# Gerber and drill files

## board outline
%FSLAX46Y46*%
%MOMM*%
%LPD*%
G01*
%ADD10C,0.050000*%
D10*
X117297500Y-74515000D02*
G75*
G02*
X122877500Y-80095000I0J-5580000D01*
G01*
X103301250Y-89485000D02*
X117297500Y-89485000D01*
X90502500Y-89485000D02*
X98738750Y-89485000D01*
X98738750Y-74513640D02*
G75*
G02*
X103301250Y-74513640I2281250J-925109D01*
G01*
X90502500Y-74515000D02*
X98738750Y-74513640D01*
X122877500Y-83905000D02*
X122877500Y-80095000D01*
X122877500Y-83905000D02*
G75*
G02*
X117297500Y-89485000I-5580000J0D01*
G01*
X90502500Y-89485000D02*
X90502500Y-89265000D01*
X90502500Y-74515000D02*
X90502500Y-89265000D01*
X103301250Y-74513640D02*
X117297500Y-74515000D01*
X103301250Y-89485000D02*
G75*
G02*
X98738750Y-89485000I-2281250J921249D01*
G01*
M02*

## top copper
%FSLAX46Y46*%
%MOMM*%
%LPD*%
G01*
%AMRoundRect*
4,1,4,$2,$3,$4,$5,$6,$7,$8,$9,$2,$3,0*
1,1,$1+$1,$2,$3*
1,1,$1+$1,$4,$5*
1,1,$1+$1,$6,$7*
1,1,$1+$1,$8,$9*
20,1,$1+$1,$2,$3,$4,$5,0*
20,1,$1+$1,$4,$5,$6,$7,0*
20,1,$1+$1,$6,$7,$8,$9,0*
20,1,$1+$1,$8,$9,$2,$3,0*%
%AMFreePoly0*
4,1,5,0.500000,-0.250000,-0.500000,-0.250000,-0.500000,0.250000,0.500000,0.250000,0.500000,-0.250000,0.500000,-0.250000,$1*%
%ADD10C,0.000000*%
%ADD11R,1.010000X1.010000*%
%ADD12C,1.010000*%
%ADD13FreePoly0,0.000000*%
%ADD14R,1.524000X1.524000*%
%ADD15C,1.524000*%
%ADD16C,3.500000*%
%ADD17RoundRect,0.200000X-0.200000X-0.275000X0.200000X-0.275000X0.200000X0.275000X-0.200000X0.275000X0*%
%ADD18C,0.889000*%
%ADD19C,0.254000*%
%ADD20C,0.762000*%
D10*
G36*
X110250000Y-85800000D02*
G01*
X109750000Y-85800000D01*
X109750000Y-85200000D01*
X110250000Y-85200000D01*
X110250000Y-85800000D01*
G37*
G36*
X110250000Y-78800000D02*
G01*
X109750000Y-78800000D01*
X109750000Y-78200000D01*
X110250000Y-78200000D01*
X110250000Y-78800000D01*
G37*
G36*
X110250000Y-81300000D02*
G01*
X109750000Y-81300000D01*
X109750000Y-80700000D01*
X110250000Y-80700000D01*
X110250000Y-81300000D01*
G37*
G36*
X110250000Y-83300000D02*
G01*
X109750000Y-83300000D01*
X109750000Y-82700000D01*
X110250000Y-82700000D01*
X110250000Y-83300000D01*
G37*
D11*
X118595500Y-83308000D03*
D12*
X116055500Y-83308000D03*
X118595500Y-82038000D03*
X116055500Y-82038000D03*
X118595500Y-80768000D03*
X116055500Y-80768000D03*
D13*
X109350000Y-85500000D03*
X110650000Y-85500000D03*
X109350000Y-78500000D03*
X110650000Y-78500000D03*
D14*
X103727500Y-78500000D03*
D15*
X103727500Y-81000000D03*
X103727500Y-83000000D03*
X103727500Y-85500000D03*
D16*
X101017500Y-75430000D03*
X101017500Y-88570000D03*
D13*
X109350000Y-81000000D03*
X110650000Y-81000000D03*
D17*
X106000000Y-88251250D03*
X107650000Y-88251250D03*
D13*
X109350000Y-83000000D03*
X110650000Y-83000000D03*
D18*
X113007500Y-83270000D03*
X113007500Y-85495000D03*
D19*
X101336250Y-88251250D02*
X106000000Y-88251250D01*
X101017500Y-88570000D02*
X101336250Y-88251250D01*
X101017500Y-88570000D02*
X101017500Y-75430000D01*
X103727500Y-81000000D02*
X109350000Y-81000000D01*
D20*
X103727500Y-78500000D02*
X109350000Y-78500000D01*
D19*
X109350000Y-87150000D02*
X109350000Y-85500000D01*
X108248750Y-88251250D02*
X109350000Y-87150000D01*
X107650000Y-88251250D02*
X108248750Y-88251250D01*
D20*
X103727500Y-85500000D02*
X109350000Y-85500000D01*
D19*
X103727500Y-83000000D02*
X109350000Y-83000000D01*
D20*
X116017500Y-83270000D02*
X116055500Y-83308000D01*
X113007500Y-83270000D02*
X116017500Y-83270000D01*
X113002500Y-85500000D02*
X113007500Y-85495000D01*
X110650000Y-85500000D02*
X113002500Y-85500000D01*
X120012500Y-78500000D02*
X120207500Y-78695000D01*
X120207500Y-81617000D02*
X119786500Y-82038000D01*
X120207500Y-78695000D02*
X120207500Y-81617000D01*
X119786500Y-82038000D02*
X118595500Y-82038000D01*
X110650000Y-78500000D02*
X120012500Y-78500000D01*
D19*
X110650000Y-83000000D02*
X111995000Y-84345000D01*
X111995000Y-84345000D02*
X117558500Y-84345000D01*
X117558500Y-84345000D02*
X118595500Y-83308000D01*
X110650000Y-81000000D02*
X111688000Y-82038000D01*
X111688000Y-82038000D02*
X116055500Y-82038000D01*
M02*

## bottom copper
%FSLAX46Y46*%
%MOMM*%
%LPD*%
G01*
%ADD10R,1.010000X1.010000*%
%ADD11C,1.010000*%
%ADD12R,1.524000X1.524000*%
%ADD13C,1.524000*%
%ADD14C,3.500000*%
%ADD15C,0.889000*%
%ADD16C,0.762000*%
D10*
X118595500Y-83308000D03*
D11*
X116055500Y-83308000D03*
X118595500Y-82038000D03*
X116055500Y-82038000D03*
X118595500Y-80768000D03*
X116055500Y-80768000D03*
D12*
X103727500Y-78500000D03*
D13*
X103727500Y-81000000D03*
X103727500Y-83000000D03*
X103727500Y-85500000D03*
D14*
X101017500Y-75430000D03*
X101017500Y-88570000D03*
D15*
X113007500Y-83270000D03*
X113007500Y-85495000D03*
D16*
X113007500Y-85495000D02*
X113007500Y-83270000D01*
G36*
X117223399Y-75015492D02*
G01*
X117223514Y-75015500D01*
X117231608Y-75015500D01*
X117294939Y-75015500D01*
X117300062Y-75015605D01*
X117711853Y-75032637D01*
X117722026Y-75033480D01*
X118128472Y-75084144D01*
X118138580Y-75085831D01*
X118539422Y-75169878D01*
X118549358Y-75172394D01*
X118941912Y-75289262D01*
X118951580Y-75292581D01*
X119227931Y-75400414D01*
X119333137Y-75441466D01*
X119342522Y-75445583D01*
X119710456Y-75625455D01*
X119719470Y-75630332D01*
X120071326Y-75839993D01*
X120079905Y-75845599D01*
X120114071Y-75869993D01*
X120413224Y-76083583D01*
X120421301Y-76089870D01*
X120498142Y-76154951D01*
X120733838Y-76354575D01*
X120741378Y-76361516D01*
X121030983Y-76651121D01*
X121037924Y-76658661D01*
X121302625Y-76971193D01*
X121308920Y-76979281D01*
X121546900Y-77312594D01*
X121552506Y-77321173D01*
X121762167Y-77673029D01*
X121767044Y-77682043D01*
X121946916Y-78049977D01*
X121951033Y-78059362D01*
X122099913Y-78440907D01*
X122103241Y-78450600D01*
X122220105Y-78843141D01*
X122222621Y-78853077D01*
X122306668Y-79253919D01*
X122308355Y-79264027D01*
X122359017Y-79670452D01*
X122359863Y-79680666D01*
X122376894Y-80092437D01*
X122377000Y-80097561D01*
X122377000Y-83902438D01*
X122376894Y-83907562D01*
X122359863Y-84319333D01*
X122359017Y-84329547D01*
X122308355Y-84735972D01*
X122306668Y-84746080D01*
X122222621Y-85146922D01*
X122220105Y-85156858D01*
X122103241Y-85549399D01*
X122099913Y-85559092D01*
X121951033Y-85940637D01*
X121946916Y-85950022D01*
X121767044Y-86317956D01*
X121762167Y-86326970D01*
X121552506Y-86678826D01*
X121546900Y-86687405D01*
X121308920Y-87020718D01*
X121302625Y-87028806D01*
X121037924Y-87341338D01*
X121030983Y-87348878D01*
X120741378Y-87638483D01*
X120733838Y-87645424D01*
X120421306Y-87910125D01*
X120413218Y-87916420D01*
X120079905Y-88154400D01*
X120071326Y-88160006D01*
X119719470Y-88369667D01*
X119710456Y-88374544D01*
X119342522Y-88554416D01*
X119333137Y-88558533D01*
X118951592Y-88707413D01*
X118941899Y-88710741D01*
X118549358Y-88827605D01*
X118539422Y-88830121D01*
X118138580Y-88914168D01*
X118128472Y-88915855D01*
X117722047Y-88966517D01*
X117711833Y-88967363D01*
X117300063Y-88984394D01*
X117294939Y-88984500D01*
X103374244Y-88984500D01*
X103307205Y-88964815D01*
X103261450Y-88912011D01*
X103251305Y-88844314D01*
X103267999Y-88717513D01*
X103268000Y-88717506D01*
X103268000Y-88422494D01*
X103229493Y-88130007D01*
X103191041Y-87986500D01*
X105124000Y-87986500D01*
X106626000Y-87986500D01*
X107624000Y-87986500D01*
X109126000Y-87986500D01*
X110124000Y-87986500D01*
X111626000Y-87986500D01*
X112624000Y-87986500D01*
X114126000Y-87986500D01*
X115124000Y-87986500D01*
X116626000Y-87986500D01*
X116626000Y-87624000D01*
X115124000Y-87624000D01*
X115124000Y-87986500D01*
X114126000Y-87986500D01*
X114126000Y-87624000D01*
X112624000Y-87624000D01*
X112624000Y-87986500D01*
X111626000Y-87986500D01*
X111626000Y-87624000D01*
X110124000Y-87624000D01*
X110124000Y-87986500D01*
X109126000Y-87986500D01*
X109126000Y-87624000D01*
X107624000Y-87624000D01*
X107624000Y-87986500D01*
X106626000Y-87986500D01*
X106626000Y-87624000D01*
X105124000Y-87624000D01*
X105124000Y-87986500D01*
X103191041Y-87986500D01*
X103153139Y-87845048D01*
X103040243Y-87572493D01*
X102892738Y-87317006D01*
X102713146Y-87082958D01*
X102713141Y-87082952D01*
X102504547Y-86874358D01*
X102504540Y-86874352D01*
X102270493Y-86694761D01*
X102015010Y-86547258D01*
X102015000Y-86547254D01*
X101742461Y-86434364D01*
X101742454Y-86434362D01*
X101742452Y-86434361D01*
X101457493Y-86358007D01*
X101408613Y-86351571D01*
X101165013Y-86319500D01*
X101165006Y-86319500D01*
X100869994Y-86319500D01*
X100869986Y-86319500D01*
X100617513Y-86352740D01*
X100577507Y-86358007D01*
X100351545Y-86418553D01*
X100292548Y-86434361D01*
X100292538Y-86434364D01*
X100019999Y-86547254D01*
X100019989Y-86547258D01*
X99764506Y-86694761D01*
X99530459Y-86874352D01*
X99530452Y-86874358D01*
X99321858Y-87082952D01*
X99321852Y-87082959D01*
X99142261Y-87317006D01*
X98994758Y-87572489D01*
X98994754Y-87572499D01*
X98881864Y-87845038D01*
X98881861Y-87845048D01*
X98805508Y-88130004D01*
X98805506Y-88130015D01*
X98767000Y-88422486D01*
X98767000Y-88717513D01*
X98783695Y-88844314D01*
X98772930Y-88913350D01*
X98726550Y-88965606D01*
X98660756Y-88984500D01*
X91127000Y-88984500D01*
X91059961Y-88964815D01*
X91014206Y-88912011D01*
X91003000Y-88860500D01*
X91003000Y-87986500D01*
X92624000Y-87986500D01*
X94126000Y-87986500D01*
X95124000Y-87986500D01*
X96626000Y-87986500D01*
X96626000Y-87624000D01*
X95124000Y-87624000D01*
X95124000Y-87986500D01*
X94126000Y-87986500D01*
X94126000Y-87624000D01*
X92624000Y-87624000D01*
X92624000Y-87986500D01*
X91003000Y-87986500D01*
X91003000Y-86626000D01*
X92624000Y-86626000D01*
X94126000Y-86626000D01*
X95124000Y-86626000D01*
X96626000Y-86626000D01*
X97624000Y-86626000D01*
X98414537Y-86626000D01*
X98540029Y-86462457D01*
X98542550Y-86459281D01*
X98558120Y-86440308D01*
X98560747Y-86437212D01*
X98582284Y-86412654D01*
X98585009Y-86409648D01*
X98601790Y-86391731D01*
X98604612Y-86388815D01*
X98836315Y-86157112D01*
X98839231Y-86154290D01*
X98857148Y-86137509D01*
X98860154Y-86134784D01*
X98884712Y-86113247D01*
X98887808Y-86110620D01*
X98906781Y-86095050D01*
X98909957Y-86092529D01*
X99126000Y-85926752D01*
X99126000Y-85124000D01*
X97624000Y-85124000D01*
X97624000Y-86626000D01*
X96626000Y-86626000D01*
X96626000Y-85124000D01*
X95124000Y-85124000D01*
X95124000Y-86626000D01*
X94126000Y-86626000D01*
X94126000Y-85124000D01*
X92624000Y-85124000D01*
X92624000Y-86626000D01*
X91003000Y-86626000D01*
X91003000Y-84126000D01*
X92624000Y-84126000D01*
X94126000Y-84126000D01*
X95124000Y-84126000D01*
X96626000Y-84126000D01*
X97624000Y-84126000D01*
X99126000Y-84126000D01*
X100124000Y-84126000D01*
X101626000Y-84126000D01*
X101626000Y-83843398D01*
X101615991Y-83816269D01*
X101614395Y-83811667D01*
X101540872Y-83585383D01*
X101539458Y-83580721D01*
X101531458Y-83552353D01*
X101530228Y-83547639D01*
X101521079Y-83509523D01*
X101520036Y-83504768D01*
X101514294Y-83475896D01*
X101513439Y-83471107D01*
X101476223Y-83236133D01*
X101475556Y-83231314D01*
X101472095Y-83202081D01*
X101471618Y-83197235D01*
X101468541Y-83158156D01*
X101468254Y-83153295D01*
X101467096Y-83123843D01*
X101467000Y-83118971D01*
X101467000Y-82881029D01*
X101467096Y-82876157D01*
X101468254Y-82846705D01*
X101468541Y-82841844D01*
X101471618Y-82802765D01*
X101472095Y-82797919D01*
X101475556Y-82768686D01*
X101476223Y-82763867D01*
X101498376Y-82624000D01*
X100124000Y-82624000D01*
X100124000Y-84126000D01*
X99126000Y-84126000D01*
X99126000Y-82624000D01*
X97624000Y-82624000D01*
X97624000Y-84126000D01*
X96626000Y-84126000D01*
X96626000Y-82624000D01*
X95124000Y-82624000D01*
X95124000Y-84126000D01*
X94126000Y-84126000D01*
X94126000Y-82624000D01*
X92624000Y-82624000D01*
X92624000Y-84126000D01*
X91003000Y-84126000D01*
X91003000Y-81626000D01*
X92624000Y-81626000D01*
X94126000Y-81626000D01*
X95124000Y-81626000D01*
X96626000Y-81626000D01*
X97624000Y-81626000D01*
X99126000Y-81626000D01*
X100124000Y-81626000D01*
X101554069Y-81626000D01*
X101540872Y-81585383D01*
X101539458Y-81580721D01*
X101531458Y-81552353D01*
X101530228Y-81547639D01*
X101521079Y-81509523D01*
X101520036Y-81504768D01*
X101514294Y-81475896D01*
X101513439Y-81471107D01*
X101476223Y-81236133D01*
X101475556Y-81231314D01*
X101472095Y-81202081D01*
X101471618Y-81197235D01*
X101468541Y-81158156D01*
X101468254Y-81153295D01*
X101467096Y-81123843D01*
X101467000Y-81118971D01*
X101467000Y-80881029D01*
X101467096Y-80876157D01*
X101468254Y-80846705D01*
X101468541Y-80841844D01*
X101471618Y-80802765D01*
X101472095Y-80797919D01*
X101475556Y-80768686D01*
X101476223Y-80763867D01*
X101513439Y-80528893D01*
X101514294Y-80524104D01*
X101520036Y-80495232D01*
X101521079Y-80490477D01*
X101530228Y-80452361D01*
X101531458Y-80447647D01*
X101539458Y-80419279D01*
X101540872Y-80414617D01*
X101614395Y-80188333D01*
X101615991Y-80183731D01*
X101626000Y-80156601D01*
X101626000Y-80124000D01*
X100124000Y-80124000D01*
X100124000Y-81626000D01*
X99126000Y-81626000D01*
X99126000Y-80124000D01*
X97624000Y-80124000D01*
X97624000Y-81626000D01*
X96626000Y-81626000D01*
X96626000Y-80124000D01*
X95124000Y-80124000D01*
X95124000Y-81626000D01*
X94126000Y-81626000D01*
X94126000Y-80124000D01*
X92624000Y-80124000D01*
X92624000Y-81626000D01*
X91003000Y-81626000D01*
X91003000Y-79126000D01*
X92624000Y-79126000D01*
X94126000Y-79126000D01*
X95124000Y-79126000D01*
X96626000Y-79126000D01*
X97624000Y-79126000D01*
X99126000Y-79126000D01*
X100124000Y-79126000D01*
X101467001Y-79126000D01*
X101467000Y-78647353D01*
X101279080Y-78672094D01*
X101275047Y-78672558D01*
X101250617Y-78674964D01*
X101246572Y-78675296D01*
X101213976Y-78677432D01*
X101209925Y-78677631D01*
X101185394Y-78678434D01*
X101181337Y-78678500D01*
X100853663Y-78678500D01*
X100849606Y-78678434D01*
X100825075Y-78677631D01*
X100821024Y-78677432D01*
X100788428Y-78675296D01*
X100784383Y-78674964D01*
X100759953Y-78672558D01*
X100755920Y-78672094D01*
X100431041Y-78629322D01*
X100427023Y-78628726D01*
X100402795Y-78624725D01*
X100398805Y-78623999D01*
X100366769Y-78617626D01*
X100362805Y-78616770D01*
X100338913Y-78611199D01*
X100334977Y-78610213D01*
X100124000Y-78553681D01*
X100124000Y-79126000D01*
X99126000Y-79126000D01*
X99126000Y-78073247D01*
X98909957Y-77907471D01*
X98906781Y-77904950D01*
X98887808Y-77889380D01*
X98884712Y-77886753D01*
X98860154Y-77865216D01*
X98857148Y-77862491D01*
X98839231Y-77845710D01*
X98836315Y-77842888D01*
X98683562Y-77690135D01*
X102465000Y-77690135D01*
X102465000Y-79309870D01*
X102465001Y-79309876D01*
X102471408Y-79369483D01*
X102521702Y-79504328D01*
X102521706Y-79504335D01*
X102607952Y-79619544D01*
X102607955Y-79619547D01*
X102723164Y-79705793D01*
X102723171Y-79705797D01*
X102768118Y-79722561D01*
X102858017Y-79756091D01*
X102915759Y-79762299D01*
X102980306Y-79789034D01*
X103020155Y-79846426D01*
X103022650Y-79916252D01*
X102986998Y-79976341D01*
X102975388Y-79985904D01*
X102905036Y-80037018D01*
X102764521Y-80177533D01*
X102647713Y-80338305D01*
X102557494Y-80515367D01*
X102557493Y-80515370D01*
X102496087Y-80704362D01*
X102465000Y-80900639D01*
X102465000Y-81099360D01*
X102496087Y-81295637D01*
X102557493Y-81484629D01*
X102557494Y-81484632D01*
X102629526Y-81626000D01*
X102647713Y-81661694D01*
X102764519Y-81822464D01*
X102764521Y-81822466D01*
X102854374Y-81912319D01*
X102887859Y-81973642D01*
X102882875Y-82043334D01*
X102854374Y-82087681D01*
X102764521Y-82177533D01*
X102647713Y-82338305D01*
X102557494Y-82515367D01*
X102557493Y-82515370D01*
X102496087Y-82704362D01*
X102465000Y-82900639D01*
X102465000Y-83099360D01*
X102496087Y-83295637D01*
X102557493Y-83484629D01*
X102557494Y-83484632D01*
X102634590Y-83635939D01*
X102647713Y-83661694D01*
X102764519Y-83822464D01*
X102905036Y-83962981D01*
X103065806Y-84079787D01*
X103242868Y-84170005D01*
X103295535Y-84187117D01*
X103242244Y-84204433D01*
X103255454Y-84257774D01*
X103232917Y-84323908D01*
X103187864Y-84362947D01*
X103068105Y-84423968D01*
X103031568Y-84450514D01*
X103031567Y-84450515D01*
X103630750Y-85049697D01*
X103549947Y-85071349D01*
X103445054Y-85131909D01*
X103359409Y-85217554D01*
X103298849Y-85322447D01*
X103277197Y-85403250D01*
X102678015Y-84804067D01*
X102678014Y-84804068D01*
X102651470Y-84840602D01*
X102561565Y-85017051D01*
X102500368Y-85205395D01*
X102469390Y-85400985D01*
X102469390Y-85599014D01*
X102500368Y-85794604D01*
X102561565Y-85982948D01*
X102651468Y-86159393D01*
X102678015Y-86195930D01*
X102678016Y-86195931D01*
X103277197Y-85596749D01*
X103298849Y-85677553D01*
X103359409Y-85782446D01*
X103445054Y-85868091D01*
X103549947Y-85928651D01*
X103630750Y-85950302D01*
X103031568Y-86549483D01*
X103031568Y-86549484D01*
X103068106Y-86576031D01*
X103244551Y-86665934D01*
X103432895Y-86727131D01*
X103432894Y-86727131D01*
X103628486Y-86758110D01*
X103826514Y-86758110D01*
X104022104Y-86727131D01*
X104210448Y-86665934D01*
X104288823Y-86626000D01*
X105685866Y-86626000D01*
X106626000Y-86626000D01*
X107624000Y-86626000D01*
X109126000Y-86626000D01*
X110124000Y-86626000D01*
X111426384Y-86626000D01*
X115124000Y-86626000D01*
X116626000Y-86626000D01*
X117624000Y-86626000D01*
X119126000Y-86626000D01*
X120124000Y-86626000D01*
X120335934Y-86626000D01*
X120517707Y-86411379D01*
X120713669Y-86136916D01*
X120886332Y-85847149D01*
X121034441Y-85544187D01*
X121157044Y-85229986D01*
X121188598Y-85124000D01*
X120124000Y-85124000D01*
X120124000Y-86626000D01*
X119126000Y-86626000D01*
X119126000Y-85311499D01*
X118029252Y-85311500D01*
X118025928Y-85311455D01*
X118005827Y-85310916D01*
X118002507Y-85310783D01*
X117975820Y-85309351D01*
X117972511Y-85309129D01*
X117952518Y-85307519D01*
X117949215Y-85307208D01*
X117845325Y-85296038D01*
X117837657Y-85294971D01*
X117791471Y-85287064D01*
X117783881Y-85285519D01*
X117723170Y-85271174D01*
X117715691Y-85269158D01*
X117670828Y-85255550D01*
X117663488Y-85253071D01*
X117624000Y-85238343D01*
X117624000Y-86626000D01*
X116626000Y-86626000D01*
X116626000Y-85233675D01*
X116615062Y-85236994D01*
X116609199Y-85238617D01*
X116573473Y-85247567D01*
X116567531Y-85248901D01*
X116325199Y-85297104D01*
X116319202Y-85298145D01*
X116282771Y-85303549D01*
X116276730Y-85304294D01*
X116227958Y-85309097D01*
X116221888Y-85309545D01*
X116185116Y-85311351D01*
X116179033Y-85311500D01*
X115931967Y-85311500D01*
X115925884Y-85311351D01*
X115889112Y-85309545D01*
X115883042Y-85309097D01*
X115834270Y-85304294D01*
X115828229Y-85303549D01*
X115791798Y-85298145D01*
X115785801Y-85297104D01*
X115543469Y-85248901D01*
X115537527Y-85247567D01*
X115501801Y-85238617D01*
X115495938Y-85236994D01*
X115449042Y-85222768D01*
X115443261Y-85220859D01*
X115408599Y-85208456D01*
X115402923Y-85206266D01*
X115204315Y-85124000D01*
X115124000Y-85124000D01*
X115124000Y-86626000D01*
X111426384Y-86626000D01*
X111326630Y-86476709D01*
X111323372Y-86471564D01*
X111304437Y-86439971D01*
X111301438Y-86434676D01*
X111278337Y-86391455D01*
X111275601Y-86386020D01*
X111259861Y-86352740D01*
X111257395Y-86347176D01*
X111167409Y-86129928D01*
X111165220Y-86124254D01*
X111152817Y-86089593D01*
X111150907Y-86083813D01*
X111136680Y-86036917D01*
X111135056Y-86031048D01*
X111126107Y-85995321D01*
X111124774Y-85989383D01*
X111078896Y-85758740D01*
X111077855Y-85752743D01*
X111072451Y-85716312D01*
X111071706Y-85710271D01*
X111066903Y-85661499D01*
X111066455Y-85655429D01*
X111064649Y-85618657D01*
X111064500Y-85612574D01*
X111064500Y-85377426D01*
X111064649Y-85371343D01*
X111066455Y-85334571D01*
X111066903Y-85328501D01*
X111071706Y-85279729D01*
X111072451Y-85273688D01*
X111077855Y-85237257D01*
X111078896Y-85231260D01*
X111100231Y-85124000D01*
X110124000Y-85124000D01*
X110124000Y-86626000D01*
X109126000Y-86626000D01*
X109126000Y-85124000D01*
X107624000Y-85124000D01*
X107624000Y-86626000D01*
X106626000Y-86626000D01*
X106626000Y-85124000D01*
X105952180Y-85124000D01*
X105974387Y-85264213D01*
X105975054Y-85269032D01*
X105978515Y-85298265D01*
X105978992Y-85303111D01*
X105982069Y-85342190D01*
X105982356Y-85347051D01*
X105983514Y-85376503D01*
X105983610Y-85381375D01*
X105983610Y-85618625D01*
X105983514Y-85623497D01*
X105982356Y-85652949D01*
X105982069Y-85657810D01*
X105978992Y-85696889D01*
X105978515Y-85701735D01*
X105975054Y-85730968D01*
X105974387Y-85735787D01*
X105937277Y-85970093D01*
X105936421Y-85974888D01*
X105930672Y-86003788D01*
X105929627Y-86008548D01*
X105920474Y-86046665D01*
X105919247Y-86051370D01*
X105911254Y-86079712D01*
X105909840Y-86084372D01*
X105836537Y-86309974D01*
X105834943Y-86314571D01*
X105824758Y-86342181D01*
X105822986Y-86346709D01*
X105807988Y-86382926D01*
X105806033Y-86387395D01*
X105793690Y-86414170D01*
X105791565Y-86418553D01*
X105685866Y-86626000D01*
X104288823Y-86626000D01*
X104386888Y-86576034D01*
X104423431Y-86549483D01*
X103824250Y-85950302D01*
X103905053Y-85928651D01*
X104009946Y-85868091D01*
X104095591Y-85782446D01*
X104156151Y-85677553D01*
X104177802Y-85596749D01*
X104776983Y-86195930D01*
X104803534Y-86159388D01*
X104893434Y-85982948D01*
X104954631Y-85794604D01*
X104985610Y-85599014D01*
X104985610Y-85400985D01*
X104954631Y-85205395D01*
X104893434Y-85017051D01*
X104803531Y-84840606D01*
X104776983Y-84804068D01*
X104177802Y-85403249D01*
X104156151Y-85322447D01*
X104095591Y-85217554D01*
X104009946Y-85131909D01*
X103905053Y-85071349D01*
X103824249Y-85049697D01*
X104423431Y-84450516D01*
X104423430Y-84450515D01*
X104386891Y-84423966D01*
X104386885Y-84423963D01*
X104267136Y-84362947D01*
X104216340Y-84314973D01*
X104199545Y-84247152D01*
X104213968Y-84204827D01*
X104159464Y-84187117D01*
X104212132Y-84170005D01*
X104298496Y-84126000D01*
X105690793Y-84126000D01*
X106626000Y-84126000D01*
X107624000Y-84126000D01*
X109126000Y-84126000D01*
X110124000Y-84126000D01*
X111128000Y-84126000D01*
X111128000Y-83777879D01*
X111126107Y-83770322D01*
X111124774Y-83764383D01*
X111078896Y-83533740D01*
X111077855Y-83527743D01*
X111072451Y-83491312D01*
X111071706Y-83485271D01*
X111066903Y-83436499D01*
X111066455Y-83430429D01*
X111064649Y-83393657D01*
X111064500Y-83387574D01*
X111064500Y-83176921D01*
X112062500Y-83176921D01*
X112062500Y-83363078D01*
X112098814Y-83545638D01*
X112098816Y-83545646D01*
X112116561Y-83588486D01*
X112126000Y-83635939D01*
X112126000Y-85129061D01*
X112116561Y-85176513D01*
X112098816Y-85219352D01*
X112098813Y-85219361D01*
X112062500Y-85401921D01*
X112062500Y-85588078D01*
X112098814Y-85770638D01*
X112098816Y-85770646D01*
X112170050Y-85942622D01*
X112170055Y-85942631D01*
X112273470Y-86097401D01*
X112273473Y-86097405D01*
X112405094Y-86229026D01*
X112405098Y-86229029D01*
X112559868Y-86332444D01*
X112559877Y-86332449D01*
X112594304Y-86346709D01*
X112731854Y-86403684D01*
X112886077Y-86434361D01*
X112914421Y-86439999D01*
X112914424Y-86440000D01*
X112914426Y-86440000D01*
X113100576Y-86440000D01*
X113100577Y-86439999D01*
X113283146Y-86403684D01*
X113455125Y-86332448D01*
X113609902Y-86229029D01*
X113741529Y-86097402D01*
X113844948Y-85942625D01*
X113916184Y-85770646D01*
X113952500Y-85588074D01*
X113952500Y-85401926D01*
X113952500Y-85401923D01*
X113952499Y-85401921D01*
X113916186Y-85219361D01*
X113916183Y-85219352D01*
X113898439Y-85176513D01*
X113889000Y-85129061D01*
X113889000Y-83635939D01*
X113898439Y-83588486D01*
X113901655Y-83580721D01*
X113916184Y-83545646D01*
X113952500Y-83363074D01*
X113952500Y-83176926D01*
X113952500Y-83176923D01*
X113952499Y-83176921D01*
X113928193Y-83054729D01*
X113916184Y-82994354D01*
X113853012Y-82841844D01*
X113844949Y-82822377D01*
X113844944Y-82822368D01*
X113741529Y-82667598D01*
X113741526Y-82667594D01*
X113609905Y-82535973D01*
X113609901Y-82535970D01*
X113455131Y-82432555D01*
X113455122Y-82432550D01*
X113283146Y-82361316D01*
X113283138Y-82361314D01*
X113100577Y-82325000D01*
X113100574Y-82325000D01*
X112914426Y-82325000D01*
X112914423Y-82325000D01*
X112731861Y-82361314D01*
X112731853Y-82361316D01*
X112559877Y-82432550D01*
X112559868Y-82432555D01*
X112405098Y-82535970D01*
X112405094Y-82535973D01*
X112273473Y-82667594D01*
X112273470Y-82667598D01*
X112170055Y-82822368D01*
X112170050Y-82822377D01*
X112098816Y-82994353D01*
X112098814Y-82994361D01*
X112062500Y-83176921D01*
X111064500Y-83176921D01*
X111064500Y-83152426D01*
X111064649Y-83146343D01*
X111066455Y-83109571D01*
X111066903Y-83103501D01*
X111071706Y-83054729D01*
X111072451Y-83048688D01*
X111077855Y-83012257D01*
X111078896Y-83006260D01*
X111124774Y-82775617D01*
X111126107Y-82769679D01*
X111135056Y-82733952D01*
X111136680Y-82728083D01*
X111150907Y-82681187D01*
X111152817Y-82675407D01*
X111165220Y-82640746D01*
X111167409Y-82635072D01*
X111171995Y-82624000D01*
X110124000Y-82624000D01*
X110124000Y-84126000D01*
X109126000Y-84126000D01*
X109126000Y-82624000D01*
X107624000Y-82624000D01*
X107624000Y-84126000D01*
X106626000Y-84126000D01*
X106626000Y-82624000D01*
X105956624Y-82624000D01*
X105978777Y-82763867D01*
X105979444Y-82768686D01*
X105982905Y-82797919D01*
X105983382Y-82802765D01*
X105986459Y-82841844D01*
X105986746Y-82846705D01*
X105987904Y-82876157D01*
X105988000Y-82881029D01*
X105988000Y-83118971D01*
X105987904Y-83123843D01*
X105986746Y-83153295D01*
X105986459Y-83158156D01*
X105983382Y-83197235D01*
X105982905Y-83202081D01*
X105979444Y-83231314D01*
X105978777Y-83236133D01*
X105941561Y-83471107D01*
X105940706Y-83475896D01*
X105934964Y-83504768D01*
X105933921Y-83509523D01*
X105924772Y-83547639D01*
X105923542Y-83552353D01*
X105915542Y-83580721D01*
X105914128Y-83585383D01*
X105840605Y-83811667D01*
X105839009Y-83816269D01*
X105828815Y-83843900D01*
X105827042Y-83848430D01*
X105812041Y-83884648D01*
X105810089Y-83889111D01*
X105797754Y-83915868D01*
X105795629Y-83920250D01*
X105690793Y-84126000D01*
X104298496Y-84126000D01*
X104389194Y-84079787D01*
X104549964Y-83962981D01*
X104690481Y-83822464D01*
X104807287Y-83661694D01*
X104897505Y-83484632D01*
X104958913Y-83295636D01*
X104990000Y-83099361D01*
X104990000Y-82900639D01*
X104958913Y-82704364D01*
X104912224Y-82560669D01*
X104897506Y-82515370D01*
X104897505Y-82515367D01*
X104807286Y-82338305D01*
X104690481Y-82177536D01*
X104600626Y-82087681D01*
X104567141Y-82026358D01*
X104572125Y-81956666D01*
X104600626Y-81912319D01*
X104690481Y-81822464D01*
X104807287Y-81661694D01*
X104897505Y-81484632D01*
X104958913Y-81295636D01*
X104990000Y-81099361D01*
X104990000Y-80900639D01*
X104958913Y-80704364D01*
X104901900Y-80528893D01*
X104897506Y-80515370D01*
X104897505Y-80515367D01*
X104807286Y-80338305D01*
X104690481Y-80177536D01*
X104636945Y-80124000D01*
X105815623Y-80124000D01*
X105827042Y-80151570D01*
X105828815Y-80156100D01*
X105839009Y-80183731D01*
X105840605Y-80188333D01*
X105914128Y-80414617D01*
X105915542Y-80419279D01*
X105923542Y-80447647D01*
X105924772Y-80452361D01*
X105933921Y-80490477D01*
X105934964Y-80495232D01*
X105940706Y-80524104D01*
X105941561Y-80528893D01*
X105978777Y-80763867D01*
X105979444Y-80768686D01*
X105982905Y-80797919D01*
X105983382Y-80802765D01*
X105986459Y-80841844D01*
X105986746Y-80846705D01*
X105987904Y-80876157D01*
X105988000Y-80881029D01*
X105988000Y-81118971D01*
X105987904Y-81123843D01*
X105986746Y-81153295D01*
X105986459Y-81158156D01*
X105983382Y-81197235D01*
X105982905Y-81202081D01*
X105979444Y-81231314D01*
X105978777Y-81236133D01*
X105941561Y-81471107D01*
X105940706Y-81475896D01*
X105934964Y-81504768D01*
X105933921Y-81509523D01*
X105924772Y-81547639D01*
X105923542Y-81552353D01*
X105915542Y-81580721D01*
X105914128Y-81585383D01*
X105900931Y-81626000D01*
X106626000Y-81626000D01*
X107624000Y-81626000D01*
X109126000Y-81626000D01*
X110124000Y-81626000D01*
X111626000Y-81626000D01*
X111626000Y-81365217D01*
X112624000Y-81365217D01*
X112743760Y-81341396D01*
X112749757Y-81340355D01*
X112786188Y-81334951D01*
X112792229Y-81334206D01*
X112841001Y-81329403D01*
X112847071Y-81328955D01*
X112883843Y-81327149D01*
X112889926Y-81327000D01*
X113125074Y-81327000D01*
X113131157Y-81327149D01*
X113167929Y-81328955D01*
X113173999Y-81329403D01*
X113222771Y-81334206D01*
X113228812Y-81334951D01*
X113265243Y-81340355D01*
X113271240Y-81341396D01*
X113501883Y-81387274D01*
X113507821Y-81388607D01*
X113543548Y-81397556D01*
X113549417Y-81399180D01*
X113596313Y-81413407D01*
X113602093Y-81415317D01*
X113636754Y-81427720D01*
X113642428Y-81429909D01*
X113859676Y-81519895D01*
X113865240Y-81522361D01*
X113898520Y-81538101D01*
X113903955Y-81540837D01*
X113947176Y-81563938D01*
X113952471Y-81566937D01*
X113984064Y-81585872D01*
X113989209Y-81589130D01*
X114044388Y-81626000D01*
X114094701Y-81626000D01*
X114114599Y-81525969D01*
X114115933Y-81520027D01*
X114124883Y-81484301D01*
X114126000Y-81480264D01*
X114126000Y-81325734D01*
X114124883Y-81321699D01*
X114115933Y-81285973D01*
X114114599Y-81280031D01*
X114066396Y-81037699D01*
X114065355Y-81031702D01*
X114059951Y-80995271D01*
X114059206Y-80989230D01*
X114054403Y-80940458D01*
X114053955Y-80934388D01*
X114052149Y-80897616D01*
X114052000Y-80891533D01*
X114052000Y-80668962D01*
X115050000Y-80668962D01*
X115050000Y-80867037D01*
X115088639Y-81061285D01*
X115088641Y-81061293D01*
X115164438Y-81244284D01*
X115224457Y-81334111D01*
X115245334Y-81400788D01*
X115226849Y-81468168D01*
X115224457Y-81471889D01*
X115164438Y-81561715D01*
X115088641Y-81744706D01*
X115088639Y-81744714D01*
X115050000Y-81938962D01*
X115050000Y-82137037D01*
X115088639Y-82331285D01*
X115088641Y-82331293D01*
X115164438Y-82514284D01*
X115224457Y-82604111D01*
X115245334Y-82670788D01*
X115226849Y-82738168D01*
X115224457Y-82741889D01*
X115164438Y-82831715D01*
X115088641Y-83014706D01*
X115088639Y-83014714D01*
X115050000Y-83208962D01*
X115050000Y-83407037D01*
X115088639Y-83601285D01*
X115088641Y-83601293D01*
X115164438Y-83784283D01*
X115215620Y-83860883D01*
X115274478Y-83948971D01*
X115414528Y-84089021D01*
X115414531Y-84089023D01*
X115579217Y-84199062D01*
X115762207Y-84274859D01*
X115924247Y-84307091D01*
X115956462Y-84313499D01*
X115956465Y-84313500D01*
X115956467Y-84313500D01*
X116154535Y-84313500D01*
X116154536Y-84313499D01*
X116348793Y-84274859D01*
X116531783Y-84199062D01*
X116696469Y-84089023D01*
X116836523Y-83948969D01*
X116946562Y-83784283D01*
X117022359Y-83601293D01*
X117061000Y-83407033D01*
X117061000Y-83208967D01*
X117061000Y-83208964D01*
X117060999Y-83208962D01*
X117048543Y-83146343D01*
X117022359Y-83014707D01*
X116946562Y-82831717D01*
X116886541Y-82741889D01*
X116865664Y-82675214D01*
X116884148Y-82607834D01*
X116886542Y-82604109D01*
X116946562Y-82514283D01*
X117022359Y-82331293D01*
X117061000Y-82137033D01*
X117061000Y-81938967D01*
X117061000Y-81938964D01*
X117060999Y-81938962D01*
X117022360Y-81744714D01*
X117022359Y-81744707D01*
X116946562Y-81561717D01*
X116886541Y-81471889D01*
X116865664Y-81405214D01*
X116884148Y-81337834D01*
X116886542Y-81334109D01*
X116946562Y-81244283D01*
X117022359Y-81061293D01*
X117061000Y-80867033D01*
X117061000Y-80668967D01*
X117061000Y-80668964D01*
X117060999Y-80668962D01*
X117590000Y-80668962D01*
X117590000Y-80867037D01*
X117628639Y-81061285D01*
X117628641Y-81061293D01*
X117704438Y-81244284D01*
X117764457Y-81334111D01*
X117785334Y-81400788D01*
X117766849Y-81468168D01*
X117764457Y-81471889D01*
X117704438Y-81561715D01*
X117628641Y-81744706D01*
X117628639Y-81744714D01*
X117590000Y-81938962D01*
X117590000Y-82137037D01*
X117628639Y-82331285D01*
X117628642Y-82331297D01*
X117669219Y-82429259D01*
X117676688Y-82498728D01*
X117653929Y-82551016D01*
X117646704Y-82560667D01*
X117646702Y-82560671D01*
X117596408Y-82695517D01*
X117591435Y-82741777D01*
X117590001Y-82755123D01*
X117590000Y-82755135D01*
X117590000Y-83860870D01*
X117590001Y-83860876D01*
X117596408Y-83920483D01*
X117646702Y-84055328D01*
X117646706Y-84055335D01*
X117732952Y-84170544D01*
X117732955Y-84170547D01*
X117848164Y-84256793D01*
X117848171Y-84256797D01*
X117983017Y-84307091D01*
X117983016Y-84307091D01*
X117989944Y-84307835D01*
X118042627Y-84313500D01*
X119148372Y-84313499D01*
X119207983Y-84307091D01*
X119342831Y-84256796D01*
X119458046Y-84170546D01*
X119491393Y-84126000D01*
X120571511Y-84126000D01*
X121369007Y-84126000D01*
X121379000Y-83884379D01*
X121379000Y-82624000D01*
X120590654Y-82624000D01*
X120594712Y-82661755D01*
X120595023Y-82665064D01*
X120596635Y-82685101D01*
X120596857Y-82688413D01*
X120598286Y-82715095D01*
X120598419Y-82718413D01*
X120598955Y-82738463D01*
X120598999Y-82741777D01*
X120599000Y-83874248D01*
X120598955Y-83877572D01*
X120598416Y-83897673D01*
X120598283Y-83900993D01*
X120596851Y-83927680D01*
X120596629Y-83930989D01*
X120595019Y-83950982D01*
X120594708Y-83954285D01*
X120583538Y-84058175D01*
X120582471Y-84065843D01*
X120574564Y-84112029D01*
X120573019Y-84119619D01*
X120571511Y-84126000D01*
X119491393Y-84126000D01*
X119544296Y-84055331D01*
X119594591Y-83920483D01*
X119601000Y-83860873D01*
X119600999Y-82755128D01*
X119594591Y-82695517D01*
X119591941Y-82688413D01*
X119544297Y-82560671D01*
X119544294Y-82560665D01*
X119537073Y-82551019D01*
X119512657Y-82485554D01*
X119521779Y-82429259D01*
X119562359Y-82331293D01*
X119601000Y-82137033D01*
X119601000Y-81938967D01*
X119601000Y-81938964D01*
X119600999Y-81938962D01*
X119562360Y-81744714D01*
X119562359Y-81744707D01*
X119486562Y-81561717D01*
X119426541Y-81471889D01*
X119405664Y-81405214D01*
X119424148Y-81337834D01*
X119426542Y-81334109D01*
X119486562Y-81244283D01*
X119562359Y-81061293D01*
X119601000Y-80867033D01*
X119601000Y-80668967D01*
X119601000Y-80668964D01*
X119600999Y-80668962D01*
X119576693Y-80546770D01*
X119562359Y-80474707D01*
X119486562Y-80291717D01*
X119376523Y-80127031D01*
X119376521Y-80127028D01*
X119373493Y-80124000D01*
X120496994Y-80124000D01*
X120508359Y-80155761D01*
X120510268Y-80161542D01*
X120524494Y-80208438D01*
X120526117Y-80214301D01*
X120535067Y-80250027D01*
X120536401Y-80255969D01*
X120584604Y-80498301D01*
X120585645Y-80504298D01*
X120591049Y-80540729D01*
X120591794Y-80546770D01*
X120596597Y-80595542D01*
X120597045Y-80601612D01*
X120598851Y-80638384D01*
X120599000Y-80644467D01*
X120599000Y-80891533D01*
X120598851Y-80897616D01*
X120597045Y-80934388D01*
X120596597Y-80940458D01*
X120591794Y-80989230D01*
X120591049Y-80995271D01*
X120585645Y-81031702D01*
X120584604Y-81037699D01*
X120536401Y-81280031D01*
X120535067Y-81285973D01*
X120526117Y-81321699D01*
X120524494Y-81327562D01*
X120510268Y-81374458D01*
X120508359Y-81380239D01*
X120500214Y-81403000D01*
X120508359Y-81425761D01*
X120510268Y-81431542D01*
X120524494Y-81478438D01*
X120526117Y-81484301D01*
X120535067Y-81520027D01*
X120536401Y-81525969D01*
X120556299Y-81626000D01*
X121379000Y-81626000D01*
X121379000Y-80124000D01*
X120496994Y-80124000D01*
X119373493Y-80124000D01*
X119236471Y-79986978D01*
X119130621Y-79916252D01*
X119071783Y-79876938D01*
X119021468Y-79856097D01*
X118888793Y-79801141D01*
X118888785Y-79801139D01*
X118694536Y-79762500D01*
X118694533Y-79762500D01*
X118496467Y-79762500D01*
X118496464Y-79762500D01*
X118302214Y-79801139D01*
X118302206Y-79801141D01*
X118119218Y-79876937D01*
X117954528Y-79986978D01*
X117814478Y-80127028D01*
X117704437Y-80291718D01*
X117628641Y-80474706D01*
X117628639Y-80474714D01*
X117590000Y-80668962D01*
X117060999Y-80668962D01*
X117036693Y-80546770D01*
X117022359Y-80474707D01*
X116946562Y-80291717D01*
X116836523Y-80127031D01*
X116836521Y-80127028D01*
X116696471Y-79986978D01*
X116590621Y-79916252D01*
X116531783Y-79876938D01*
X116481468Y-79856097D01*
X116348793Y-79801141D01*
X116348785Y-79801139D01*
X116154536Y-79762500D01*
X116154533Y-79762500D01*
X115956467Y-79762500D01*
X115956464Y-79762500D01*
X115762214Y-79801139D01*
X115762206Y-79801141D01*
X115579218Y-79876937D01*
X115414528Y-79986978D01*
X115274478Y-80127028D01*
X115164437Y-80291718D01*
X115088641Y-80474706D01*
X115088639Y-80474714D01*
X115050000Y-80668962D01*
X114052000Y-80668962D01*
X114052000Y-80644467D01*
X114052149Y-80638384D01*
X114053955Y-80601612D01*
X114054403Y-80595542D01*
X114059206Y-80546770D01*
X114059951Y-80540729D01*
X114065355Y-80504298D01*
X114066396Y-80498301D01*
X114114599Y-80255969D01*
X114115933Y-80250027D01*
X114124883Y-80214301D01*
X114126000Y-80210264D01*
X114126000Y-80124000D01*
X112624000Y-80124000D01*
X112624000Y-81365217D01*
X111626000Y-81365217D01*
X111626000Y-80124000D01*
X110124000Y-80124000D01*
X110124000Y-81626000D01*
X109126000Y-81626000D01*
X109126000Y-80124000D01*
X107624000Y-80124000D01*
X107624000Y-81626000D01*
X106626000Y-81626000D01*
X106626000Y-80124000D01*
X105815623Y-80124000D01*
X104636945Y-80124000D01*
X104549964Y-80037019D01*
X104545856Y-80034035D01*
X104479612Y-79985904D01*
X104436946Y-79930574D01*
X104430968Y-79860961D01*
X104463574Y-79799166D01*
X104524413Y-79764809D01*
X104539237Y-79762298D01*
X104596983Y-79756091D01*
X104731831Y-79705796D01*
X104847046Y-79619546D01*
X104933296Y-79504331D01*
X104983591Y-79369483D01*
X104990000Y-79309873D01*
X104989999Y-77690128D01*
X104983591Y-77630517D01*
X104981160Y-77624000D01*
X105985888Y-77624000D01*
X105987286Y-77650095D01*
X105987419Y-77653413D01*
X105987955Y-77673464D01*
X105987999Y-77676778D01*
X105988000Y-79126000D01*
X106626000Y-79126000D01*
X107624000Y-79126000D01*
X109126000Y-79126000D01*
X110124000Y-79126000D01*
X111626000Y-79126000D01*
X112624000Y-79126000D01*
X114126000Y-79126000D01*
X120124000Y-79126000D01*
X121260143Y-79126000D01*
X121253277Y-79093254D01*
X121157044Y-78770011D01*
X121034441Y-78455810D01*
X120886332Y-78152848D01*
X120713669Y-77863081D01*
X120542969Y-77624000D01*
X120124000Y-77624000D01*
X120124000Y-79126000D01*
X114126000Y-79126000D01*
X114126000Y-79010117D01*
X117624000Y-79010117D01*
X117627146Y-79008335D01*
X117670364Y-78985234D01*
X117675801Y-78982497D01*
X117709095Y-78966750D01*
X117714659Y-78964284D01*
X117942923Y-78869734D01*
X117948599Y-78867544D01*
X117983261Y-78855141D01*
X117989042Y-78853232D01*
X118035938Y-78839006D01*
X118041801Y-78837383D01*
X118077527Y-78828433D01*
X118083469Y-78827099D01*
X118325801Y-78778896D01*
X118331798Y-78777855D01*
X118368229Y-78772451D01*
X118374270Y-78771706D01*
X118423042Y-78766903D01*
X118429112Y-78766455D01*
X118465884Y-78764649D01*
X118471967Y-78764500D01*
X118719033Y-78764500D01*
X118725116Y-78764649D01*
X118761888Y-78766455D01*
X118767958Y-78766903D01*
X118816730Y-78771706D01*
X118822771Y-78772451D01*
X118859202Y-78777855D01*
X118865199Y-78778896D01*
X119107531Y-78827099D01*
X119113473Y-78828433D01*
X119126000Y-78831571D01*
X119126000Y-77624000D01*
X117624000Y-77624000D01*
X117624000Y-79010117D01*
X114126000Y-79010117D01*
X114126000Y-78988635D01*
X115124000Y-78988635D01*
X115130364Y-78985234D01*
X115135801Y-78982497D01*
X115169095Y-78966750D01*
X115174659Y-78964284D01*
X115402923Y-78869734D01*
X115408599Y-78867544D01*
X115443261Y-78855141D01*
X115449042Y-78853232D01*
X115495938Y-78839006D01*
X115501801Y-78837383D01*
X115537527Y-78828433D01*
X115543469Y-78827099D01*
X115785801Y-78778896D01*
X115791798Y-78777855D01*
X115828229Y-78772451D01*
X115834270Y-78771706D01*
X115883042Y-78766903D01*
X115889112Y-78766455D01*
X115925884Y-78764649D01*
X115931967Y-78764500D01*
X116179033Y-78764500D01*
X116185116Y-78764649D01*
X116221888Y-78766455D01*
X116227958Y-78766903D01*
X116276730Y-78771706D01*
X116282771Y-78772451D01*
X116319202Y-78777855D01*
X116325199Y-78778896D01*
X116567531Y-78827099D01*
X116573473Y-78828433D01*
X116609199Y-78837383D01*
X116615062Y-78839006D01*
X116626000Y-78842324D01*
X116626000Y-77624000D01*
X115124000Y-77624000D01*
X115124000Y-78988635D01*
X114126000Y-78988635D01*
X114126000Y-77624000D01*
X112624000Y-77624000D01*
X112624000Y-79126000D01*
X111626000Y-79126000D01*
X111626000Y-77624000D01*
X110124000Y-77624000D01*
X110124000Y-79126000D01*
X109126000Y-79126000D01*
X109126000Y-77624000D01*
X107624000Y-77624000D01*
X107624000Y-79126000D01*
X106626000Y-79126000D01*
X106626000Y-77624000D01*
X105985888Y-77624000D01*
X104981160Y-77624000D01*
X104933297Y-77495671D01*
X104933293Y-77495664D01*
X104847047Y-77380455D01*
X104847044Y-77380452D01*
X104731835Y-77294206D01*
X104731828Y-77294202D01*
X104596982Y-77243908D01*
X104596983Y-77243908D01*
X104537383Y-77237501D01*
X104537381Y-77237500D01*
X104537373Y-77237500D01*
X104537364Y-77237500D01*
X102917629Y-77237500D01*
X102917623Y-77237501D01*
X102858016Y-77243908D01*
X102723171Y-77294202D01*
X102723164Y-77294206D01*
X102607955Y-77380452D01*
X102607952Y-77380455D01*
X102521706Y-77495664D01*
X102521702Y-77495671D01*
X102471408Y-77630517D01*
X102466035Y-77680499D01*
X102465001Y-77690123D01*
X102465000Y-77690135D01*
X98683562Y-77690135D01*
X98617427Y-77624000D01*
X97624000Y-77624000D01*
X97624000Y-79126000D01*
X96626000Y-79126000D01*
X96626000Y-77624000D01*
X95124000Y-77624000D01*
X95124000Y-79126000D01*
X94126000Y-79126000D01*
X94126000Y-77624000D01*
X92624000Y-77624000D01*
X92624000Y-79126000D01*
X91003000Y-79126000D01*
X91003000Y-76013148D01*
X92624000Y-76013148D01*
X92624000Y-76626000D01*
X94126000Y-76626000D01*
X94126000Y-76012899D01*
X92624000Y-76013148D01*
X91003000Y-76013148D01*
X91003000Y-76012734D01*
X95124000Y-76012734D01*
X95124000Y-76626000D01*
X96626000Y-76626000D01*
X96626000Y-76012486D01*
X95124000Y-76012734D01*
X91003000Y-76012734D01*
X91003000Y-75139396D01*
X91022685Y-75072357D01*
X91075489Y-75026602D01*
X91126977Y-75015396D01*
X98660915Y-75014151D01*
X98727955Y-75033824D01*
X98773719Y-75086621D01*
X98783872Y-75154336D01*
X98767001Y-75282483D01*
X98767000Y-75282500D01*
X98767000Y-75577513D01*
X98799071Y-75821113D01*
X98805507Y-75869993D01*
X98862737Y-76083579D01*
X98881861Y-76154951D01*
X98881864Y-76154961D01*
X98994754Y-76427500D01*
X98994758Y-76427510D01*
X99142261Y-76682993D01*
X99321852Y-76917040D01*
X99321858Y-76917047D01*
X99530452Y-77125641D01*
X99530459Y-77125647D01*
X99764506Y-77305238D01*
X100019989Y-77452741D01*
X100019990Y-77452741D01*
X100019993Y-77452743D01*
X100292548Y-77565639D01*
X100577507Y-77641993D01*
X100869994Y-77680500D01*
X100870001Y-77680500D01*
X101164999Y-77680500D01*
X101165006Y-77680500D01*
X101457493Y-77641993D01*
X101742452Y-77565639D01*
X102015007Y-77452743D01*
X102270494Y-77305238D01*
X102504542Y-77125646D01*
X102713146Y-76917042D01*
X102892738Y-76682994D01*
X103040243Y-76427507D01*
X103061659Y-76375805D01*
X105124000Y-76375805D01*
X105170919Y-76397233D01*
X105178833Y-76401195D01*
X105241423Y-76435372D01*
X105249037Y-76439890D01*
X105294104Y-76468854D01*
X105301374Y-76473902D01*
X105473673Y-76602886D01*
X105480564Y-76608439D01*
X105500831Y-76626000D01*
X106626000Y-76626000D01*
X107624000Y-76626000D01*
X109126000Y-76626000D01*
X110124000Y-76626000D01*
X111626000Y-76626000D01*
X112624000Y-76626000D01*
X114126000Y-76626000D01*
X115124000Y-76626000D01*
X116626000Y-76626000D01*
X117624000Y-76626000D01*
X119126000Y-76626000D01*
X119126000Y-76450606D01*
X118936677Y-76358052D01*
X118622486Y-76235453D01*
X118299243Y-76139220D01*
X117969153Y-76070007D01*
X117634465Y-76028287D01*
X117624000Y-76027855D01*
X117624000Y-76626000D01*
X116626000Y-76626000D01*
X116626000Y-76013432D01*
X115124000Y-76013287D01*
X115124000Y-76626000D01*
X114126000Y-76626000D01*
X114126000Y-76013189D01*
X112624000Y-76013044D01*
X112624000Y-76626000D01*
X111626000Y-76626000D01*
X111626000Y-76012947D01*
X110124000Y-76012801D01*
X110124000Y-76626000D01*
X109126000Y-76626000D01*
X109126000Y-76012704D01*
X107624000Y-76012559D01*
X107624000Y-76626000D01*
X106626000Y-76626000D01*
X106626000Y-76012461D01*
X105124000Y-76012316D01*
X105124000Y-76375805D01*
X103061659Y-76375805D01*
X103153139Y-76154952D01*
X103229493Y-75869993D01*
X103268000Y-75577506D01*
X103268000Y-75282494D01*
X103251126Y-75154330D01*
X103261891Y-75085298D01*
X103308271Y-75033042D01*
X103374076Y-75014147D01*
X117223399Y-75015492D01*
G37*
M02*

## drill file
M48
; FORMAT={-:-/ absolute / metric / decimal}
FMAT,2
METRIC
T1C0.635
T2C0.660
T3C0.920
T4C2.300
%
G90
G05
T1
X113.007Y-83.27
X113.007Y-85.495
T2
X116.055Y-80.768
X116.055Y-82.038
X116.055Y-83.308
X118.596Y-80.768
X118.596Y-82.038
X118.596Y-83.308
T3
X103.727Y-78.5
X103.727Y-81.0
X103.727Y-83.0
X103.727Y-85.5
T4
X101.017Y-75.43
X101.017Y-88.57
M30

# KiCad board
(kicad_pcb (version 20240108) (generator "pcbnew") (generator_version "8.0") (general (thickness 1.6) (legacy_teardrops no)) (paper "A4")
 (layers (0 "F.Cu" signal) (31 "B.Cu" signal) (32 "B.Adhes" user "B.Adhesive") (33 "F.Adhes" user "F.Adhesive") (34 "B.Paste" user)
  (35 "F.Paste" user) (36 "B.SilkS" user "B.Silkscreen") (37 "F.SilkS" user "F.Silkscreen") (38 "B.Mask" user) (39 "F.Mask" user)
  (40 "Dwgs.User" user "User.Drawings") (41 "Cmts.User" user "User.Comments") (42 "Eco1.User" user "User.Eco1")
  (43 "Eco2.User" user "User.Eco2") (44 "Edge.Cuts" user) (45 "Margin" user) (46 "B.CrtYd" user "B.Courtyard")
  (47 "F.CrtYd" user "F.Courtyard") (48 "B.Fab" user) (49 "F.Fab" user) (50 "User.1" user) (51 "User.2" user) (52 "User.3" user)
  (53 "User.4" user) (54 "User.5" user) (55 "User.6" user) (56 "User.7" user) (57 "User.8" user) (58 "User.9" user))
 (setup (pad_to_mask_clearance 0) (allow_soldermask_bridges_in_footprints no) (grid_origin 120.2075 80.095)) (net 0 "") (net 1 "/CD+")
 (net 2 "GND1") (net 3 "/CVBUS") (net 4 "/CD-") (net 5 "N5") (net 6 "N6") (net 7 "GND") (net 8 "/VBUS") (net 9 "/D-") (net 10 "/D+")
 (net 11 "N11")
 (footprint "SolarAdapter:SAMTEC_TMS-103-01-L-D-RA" (layer "F.Cu") (at 117.3255 82.038 -90)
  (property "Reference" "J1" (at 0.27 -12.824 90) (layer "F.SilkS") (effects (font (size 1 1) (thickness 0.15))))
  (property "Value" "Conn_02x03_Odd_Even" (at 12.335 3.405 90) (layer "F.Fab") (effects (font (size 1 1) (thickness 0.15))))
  (pad "1" thru_hole rect (at 1.27 -1.27 270) (size 1.01 1.01) (drill 0.66) (layers "*.Cu" "*.Mask") (remove_unused_layers no)
   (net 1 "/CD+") (solder_mask_margin 0.102))
  (pad "2" thru_hole circle (at 1.27 1.27 270) (size 1.01 1.01) (drill 0.66) (layers "*.Cu" "*.Mask") (remove_unused_layers no)
   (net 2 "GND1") (solder_mask_margin 0.102))
  (pad "3" thru_hole circle (at 0 -1.27 270) (size 1.01 1.01) (drill 0.66) (layers "*.Cu" "*.Mask") (remove_unused_layers no)
   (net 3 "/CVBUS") (solder_mask_margin 0.102))
  (pad "4" thru_hole circle (at 0 1.27 270) (size 1.01 1.01) (drill 0.66) (layers "*.Cu" "*.Mask") (remove_unused_layers no) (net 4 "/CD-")
   (solder_mask_margin 0.102))
  (pad "5" thru_hole circle (at -1.27 -1.27 270) (size 1.01 1.01) (drill 0.66) (layers "*.Cu" "*.Mask") (remove_unused_layers no)
   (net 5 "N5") (solder_mask_margin 0.102))
  (pad "6" thru_hole circle (at -1.27 1.27 270) (size 1.01 1.01) (drill 0.66) (layers "*.Cu" "*.Mask") (remove_unused_layers no)
   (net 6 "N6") (solder_mask_margin 0.102)))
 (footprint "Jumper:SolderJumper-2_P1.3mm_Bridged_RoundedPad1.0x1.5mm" (layer "F.Cu") (at 110 85.5)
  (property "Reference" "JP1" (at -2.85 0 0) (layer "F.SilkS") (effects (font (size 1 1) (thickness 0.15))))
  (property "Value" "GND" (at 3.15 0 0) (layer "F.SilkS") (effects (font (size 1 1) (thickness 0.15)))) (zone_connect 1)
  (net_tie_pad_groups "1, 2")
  (fp_poly (pts (xy 0.25 -0.3) (xy -0.25 -0.3) (xy -0.25 0.3) (xy 0.25 0.3)) (stroke (width 0) (type solid)) (fill solid) (layer "F.Cu"))
  (pad "1" smd custom (at -0.65 0) (size 1 0.5) (layers "F.Cu" "F.Mask") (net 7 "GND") (zone_connect 2) (thermal_bridge_angle 45)
   (options (clearance outline) (anchor rect)) (primitives))
  (pad "2" smd custom (at 0.65 0) (size 1 0.5) (layers "F.Cu" "F.Mask") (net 2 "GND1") (zone_connect 2) (thermal_bridge_angle 45)
   (options (clearance outline) (anchor rect)) (primitives)))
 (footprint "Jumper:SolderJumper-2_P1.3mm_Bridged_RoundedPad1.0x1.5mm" (layer "F.Cu") (at 110 78.5)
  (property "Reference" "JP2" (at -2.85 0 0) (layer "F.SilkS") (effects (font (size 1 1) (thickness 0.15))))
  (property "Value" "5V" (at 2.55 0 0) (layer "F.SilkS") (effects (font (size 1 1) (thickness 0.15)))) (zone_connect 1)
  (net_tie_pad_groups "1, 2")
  (fp_poly (pts (xy 0.25 -0.3) (xy -0.25 -0.3) (xy -0.25 0.3) (xy 0.25 0.3)) (stroke (width 0) (type solid)) (fill solid) (layer "F.Cu"))
  (pad "1" smd custom (at -0.65 0) (size 1 0.5) (layers "F.Cu" "F.Mask") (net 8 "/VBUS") (zone_connect 2) (thermal_bridge_angle 45)
   (options (clearance outline) (anchor rect)) (primitives))
  (pad "2" smd custom (at 0.65 0) (size 1 0.5) (layers "F.Cu" "F.Mask") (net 3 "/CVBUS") (zone_connect 2) (thermal_bridge_angle 45)
   (options (clearance outline) (anchor rect)) (primitives)))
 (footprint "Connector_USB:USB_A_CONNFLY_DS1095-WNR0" (layer "F.Cu") (at 103.7275 78.5 -90)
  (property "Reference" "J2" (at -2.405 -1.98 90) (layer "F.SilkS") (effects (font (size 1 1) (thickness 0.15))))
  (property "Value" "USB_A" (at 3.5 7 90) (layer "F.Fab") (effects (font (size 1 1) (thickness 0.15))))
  (pad "1" thru_hole rect (at 0 0 270) (size 1.524 1.524) (drill 0.92) (layers "*.Cu" "*.Mask") (remove_unused_layers no) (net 8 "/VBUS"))
  (pad "2" thru_hole circle (at 2.5 0 270) (size 1.524 1.524) (drill 0.92) (layers "*.Cu" "*.Mask") (remove_unused_layers no) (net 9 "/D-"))
  (pad "3" thru_hole circle (at 4.5 0 270) (size 1.524 1.524) (drill 0.92) (layers "*.Cu" "*.Mask") (remove_unused_layers no) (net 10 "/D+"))
  (pad "4" thru_hole circle (at 7 0 270) (size 1.524 1.524) (drill 0.92) (layers "*.Cu" "*.Mask") (remove_unused_layers no) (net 7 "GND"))
  (pad "5" thru_hole circle (at -3.07 2.71 270) (size 3.5 3.5) (drill 2.3) (layers "*.Cu" "*.Mask") (remove_unused_layers no) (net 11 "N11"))
  (pad "5" thru_hole circle (at 10.07 2.71 270) (size 3.5 3.5) (drill 2.3) (layers "*.Cu" "*.Mask") (remove_unused_layers no) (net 11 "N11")))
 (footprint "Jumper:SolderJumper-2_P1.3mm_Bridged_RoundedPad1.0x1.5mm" (layer "F.Cu") (at 110 81)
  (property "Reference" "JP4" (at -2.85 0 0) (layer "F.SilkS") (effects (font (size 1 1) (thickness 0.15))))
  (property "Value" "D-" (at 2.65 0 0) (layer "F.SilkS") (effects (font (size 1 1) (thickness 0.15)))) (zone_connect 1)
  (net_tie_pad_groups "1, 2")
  (fp_poly (pts (xy 0.25 -0.3) (xy -0.25 -0.3) (xy -0.25 0.3) (xy 0.25 0.3)) (stroke (width 0) (type solid)) (fill solid) (layer "F.Cu"))
  (pad "1" smd custom (at -0.65 0) (size 1 0.5) (layers "F.Cu" "F.Mask") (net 9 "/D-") (zone_connect 2) (thermal_bridge_angle 45)
   (options (clearance outline) (anchor rect)) (primitives))
  (pad "2" smd custom (at 0.65 0) (size 1 0.5) (layers "F.Cu" "F.Mask") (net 4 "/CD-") (zone_connect 2) (thermal_bridge_angle 45)
   (options (clearance outline) (anchor rect)) (primitives)))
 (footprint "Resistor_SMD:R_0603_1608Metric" (layer "F.Cu") (at 106.825 88.25125)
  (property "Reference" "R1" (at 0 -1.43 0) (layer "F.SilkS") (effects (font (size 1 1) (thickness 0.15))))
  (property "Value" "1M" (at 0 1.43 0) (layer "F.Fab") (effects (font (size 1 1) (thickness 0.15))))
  (pad "1" smd roundrect (at -0.825 0) (size 0.8 0.95) (layers "F.Cu" "F.Paste" "F.Mask") (roundrect_rratio 0.25) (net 11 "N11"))
  (pad "2" smd roundrect (at 0.825 0) (size 0.8 0.95) (layers "F.Cu" "F.Paste" "F.Mask") (roundrect_rratio 0.25) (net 7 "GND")))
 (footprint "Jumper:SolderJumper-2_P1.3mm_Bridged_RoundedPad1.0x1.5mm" (layer "F.Cu") (at 110 83)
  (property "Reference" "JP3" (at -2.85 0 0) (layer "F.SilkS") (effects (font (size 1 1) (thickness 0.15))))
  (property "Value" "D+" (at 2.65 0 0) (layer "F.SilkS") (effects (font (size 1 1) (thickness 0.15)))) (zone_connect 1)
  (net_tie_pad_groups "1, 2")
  (fp_poly (pts (xy 0.25 -0.3) (xy -0.25 -0.3) (xy -0.25 0.3) (xy 0.25 0.3)) (stroke (width 0) (type solid)) (fill solid) (layer "F.Cu"))
  (pad "1" smd custom (at -0.65 0) (size 1 0.5) (layers "F.Cu" "F.Mask") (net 10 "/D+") (zone_connect 2) (thermal_bridge_angle 45)
   (options (clearance outline) (anchor rect)) (primitives))
  (pad "2" smd custom (at 0.65 0) (size 1 0.5) (layers "F.Cu" "F.Mask") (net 1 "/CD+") (zone_connect 2) (thermal_bridge_angle 45)
   (options (clearance outline) (anchor rect)) (primitives)))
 (gr_arc (start 117.2975 74.515) (mid 121.243156 76.149344) (end 122.8775 80.095) (stroke (width 0.05) (type default)) (layer "Edge.Cuts"))
 (gr_line (start 103.30125 89.485) (end 117.2975 89.485) (stroke (width 0.05) (type default)) (layer "Edge.Cuts"))
 (gr_line (start 90.5025 89.485) (end 98.73875 89.485) (stroke (width 0.05) (type default)) (layer "Edge.Cuts"))
 (gr_arc (start 98.73875 74.51364) (mid 101.02 72.977057) (end 103.30125 74.51364) (stroke (width 0.05) (type default)) (layer "Edge.Cuts"))
 (gr_line (start 90.5025 74.515) (end 98.73875 74.51364) (stroke (width 0.05) (type default)) (layer "Edge.Cuts"))
 (gr_line (start 122.8775 83.905) (end 122.8775 80.095) (stroke (width 0.05) (type default)) (layer "Edge.Cuts"))
 (gr_arc (start 122.8775 83.905) (mid 121.243156 87.850656) (end 117.2975 89.485) (stroke (width 0.05) (type default)) (layer "Edge.Cuts"))
 (gr_line (start 90.5025 89.485) (end 90.5025 89.265) (stroke (width 0.05) (type default)) (layer "Edge.Cuts"))
 (gr_line (start 90.5025 74.515) (end 90.5025 89.265) (stroke (width 0.05) (type default)) (layer "Edge.Cuts"))
 (gr_line (start 103.30125 74.51364) (end 117.2975 74.515) (stroke (width 0.05) (type default)) (layer "Edge.Cuts"))
 (gr_arc (start 103.30125 89.485) (mid 101.02 91.023995) (end 98.73875 89.485) (stroke (width 0.05) (type default)) (layer "Edge.Cuts"))
 (segment (start 101.33625 88.25125) (end 106 88.25125) (width 0.254) (layer "F.Cu") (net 11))
 (segment (start 101.0175 88.57) (end 101.33625 88.25125) (width 0.254) (layer "F.Cu") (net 11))
 (segment (start 101.0175 88.57) (end 101.0175 75.43) (width 0.254) (layer "F.Cu") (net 11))
 (segment (start 103.7275 81) (end 109.35 81) (width 0.254) (layer "F.Cu") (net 9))
 (segment (start 103.7275 78.5) (end 109.35 78.5) (width 0.762) (layer "F.Cu") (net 8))
 (segment (start 109.35 87.15) (end 109.35 85.5) (width 0.254) (layer "F.Cu") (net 7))
 (segment (start 108.24875 88.25125) (end 109.35 87.15) (width 0.254) (layer "F.Cu") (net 7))
 (segment (start 107.65 88.25125) (end 108.24875 88.25125) (width 0.254) (layer "F.Cu") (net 7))
 (segment (start 103.7275 85.5) (end 109.35 85.5) (width 0.762) (layer "F.Cu") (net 7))
 (segment (start 103.7275 83) (end 109.35 83) (width 0.254) (layer "F.Cu") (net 10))
 (segment (start 116.0175 83.27) (end 116.0555 83.308) (width 0.762) (layer "F.Cu") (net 2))
 (segment (start 113.0075 83.27) (end 116.0175 83.27) (width 0.762) (layer "F.Cu") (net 2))
 (segment (start 113.0025 85.5) (end 113.0075 85.495) (width 0.762) (layer "F.Cu") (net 2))
 (segment (start 110.65 85.5) (end 113.0025 85.5) (width 0.762) (layer "F.Cu") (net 2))
 (via (at 113.0075 83.27) (size 0.889) (drill 0.635) (layers "F.Cu" "B.Cu") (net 2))
 (via (at 113.0075 85.495) (size 0.889) (drill 0.635) (layers "F.Cu" "B.Cu") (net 2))
 (segment (start 113.0075 85.495) (end 113.0075 83.27) (width 0.762) (layer "B.Cu") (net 2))
 (segment (start 120.0125 78.5) (end 120.2075 78.695) (width 0.762) (layer "F.Cu") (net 3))
 (segment (start 120.2075 81.617) (end 119.7865 82.038) (width 0.762) (layer "F.Cu") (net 3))
 (segment (start 120.2075 78.695) (end 120.2075 81.617) (width 0.762) (layer "F.Cu") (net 3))
 (segment (start 119.7865 82.038) (end 118.5955 82.038) (width 0.762) (layer "F.Cu") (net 3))
 (segment (start 110.65 78.5) (end 120.0125 78.5) (width 0.762) (layer "F.Cu") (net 3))
 (segment (start 110.65 83) (end 111.995 84.345) (width 0.254) (layer "F.Cu") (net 1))
 (segment (start 111.995 84.345) (end 117.5585 84.345) (width 0.254) (layer "F.Cu") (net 1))
 (segment (start 117.5585 84.345) (end 118.5955 83.308) (width 0.254) (layer "F.Cu") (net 1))
 (segment (start 110.65 81) (end 111.688 82.038) (width 0.254) (layer "F.Cu") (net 4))
 (segment (start 111.688 82.038) (end 116.0555 82.038) (width 0.254) (layer "F.Cu") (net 4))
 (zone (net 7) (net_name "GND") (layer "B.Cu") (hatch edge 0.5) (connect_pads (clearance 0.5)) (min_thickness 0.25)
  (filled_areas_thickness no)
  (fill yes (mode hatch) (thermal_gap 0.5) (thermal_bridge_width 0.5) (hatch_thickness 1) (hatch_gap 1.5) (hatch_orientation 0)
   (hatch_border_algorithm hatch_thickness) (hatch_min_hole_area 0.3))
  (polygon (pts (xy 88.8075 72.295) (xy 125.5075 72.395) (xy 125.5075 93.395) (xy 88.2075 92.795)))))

